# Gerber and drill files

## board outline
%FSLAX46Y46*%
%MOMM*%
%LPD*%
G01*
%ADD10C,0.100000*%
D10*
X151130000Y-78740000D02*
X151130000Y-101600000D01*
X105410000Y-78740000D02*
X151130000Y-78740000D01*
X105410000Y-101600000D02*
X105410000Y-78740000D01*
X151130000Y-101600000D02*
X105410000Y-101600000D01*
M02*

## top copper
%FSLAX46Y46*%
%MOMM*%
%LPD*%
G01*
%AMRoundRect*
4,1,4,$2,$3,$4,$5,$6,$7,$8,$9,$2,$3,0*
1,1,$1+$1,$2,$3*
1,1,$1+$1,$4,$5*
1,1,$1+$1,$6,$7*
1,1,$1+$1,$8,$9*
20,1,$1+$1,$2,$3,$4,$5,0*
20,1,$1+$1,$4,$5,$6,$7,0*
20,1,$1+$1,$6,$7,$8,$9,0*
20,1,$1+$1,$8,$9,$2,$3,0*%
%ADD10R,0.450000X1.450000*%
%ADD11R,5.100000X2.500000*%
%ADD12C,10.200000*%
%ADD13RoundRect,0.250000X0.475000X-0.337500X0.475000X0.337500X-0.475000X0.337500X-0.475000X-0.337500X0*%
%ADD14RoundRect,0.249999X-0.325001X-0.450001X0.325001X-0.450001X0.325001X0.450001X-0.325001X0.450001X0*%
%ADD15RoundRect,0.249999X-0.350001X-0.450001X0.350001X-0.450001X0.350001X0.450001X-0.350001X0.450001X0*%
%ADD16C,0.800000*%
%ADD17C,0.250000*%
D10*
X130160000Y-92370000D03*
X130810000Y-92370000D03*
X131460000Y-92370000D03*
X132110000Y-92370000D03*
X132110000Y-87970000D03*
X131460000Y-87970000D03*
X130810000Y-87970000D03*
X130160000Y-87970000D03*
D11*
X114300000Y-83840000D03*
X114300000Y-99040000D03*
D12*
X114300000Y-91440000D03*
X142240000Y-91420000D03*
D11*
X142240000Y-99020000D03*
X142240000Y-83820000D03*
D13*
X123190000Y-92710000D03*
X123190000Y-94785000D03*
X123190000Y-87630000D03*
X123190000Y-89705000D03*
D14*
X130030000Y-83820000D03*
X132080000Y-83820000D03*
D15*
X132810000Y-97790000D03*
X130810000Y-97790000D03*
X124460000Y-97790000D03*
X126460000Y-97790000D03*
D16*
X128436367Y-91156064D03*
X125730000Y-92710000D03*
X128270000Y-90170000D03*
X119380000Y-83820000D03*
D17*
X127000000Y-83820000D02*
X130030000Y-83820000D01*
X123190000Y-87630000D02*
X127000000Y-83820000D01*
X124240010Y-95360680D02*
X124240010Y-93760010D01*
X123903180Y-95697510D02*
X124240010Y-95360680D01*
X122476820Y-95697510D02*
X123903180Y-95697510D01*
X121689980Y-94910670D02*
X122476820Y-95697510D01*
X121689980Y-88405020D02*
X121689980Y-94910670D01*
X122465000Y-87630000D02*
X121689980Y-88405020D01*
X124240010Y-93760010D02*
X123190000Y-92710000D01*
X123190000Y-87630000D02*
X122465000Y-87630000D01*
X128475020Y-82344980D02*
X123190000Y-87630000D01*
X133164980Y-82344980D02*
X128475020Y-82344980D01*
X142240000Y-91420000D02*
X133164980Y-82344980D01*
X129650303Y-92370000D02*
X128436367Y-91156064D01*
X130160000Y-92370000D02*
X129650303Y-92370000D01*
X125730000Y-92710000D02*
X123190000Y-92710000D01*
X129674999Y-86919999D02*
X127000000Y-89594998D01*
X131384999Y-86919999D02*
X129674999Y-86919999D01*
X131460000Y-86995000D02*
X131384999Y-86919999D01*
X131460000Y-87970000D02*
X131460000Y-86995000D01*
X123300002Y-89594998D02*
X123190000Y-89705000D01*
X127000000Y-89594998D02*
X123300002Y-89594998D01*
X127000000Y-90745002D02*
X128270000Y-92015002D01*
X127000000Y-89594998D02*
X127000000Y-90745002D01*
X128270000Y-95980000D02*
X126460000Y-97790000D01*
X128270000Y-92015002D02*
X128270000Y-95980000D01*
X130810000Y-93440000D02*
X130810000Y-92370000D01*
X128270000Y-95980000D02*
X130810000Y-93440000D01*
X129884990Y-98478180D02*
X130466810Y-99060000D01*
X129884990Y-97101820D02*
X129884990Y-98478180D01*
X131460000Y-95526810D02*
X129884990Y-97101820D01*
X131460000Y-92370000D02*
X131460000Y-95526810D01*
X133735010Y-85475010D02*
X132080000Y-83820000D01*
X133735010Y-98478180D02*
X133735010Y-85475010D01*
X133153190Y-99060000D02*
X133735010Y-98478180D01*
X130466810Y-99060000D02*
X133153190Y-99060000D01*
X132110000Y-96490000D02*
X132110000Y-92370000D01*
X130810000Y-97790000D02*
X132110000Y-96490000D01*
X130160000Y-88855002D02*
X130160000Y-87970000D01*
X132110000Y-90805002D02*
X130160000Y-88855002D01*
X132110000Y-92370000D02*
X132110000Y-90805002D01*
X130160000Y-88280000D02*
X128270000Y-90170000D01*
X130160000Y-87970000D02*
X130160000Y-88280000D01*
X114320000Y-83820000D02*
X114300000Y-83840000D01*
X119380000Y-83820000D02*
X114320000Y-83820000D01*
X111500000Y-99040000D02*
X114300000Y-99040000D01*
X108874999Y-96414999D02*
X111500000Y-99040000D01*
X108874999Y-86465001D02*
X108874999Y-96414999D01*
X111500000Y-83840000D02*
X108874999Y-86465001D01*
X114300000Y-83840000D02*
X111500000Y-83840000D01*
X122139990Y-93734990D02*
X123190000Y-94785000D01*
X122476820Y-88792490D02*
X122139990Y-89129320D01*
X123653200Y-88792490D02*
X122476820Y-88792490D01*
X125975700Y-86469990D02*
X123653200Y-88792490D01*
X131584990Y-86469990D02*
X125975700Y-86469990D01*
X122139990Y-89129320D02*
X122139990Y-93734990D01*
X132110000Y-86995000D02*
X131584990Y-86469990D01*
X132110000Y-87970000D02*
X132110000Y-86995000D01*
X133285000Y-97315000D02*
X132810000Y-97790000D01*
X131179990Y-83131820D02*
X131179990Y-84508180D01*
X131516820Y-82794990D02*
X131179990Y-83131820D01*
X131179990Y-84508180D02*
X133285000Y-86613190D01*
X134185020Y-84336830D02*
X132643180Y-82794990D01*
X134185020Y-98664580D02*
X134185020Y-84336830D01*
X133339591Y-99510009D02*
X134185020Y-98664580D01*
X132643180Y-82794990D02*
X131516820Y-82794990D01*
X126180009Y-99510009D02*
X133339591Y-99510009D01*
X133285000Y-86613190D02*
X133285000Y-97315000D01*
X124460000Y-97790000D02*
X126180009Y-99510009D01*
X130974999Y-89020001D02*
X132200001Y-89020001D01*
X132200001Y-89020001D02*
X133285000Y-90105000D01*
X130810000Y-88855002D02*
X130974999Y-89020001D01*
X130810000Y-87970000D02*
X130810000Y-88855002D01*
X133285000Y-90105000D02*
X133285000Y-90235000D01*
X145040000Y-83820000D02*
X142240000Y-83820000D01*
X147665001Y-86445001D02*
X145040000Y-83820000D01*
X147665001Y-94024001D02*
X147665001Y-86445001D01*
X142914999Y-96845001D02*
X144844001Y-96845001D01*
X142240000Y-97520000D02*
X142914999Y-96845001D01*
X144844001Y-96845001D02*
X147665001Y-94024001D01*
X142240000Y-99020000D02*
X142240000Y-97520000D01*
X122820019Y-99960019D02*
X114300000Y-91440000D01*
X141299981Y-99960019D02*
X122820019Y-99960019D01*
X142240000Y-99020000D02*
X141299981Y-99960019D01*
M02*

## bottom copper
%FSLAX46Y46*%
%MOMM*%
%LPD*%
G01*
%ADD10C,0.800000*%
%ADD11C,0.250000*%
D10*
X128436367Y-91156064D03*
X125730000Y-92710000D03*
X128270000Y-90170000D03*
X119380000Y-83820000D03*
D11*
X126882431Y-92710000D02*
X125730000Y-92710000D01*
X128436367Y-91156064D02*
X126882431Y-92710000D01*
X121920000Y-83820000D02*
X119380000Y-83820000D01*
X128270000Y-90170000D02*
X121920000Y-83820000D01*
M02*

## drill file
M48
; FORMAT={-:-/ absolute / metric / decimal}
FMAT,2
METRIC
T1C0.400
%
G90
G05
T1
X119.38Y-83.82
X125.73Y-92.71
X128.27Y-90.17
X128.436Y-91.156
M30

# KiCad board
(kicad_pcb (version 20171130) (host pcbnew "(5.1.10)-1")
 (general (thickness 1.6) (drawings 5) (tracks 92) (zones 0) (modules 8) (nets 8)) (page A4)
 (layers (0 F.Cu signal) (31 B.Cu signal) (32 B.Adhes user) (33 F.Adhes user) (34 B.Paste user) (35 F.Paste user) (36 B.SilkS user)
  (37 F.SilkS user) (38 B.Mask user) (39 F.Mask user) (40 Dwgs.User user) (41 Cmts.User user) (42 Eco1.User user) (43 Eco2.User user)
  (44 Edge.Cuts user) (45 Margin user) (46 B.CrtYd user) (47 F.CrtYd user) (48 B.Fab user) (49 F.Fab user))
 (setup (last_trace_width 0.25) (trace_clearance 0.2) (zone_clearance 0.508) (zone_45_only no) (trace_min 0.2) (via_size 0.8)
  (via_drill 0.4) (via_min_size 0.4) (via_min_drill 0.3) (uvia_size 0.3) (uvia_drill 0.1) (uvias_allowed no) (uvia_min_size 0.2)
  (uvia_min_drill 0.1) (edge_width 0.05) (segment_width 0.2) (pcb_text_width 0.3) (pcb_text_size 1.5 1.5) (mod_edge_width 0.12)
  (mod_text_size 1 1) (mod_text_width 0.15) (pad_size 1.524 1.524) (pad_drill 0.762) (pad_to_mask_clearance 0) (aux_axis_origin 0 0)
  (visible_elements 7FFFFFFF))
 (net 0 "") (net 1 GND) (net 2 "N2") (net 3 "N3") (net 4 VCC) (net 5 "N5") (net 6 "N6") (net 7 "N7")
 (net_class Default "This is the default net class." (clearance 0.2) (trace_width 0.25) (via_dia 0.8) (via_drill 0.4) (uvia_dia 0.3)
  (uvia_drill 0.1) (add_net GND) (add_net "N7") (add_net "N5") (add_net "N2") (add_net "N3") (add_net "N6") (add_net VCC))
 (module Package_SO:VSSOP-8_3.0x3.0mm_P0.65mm (layer F.Cu) (at 131.135 90.17 90)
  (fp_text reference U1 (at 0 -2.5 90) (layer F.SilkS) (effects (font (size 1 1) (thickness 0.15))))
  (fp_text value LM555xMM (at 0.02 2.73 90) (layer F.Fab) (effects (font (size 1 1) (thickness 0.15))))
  (pad 1 smd rect (at -2.2 -0.975) (size 0.45 1.45) (layers F.Cu F.Paste F.Mask) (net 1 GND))
  (pad 2 smd rect (at -2.2 -0.325) (size 0.45 1.45) (layers F.Cu F.Paste F.Mask) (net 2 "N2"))
  (pad 3 smd rect (at -2.2 0.325) (size 0.45 1.45) (layers F.Cu F.Paste F.Mask) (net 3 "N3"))
  (pad 4 smd rect (at -2.2 0.975) (size 0.45 1.45) (layers F.Cu F.Paste F.Mask) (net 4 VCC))
  (pad 5 smd rect (at 2.2 0.975) (size 0.45 1.45) (layers F.Cu F.Paste F.Mask) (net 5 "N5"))
  (pad 6 smd rect (at 2.2 0.325) (size 0.45 1.45) (layers F.Cu F.Paste F.Mask) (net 2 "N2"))
  (pad 7 smd rect (at 2.2 -0.325) (size 0.45 1.45) (layers F.Cu F.Paste F.Mask) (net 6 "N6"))
  (pad 8 smd rect (at 2.2 -0.975) (size 0.45 1.45) (layers F.Cu F.Paste F.Mask) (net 4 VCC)))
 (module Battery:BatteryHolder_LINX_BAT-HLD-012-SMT (layer F.Cu) (at 114.3 91.44 270)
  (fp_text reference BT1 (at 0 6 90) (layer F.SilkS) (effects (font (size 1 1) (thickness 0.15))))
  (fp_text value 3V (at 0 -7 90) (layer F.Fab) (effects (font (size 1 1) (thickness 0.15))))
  (pad 1 smd rect (at -7.6 0 270) (size 2.5 5.1) (layers F.Cu F.Paste F.Mask) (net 4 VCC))
  (pad 1 smd rect (at 7.6 0 270) (size 2.5 5.1) (layers F.Cu F.Paste F.Mask) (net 4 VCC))
  (pad 2 smd circle (at 0 0 270) (size 10.2 10.2) (layers F.Cu F.Mask) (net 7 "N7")))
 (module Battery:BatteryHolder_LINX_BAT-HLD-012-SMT (layer F.Cu) (at 142.24 91.42 270)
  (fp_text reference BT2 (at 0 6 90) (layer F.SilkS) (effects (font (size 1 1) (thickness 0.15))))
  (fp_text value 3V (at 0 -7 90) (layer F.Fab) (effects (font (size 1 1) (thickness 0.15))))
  (pad 2 smd circle (at 0 0 270) (size 10.2 10.2) (layers F.Cu F.Mask) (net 1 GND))
  (pad 1 smd rect (at 7.6 0 270) (size 2.5 5.1) (layers F.Cu F.Paste F.Mask) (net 7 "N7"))
  (pad 1 smd rect (at -7.6 0 270) (size 2.5 5.1) (layers F.Cu F.Paste F.Mask) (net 7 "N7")))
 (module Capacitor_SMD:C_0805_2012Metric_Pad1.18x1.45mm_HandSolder (layer F.Cu) (at 123.19 93.7475 90)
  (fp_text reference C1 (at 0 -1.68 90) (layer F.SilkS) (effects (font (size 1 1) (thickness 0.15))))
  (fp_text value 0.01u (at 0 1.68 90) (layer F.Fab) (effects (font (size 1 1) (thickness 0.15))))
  (pad 2 smd roundrect (at 1.0375 0 90) (size 1.175 1.45) (layers F.Cu F.Paste F.Mask) (roundrect_rratio 0.2127659574468085) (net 1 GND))
  (pad 1 smd roundrect (at -1.0375 0 90) (size 1.175 1.45) (layers F.Cu F.Paste F.Mask) (roundrect_rratio 0.2127659574468085) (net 5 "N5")))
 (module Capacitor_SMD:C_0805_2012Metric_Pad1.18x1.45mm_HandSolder (layer F.Cu) (at 123.19 88.6675 90)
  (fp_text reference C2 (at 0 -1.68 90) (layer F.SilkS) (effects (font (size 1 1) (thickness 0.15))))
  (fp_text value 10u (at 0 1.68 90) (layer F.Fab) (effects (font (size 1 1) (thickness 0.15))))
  (pad 2 smd roundrect (at 1.0375 0 90) (size 1.175 1.45) (layers F.Cu F.Paste F.Mask) (roundrect_rratio 0.2127659574468085) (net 1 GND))
  (pad 1 smd roundrect (at -1.0375 0 90) (size 1.175 1.45) (layers F.Cu F.Paste F.Mask) (roundrect_rratio 0.2127659574468085) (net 2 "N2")))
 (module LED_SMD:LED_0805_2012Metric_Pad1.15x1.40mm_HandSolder (layer F.Cu) (at 131.055 83.82)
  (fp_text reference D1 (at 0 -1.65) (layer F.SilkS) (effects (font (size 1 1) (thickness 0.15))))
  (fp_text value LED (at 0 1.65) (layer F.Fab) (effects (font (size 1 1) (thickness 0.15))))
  (pad 1 smd roundrect (at -1.025 0) (size 1.15 1.4) (layers F.Cu F.Paste F.Mask) (roundrect_rratio 0.2173904347826087) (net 1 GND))
  (pad 2 smd roundrect (at 1.025 0) (size 1.15 1.4) (layers F.Cu F.Paste F.Mask) (roundrect_rratio 0.2173904347826087) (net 3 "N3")))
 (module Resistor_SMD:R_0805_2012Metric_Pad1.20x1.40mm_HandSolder (layer F.Cu) (at 131.81 97.79)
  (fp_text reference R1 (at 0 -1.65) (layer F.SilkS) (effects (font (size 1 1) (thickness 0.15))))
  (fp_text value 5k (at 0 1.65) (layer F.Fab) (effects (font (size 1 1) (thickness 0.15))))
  (pad 2 smd roundrect (at 1 0) (size 1.2 1.4) (layers F.Cu F.Paste F.Mask) (roundrect_rratio 0.2083325) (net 6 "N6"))
  (pad 1 smd roundrect (at -1 0) (size 1.2 1.4) (layers F.Cu F.Paste F.Mask) (roundrect_rratio 0.2083325) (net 4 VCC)))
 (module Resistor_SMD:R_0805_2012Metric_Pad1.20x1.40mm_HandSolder (layer F.Cu) (at 125.46 97.79)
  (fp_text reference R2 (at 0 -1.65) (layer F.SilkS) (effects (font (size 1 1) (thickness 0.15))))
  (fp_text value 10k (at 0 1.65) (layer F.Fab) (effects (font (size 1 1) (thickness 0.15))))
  (pad 1 smd roundrect (at -1 0) (size 1.2 1.4) (layers F.Cu F.Paste F.Mask) (roundrect_rratio 0.2083325) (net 6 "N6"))
  (pad 2 smd roundrect (at 1 0) (size 1.2 1.4) (layers F.Cu F.Paste F.Mask) (roundrect_rratio 0.2083325) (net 2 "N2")))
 (gr_line (start 151.13 78.74) (end 151.13 101.6) (layer Edge.Cuts) (width 0.1))
 (gr_line (start 105.41 78.74) (end 151.13 78.74) (layer Edge.Cuts) (width 0.1))
 (gr_line (start 105.41 101.6) (end 105.41 78.74) (layer Edge.Cuts) (width 0.1))
 (gr_line (start 151.13 101.6) (end 105.41 101.6) (layer Edge.Cuts) (width 0.1))
 (segment (start 127 83.82) (end 130.03 83.82) (width 0.25) (layer F.Cu) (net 1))
 (segment (start 123.19 87.63) (end 127 83.82) (width 0.25) (layer F.Cu) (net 1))
 (segment (start 124.24001 95.36068) (end 124.24001 93.76001) (width 0.25) (layer F.Cu) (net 1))
 (segment (start 123.90318 95.69751) (end 124.24001 95.36068) (width 0.25) (layer F.Cu) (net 1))
 (segment (start 122.47682 95.69751) (end 123.90318 95.69751) (width 0.25) (layer F.Cu) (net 1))
 (segment (start 121.68998 94.91067) (end 122.47682 95.69751) (width 0.25) (layer F.Cu) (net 1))
 (segment (start 121.68998 88.40502) (end 121.68998 94.91067) (width 0.25) (layer F.Cu) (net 1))
 (segment (start 122.465 87.63) (end 121.68998 88.40502) (width 0.25) (layer F.Cu) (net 1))
 (segment (start 124.24001 93.76001) (end 123.19 92.71) (width 0.25) (layer F.Cu) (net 1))
 (segment (start 123.19 87.63) (end 122.465 87.63) (width 0.25) (layer F.Cu) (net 1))
 (segment (start 128.47502 82.34498) (end 123.19 87.63) (width 0.25) (layer F.Cu) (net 1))
 (segment (start 133.16498 82.34498) (end 128.47502 82.34498) (width 0.25) (layer F.Cu) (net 1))
 (segment (start 142.24 91.42) (end 133.16498 82.34498) (width 0.25) (layer F.Cu) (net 1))
 (via (at 128.436367 91.156064) (size 0.8) (drill 0.4) (layers F.Cu B.Cu) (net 1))
 (segment (start 129.650303 92.37) (end 128.436367 91.156064) (width 0.25) (layer F.Cu) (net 1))
 (segment (start 130.16 92.37) (end 129.650303 92.37) (width 0.25) (layer F.Cu) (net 1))
 (via (at 125.73 92.71) (size 0.8) (drill 0.4) (layers F.Cu B.Cu) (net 1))
 (segment (start 126.882431 92.71) (end 125.73 92.71) (width 0.25) (layer B.Cu) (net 1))
 (segment (start 128.436367 91.156064) (end 126.882431 92.71) (width 0.25) (layer B.Cu) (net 1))
 (segment (start 125.73 92.71) (end 123.19 92.71) (width 0.25) (layer F.Cu) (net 1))
 (segment (start 129.674999 86.919999) (end 127 89.594998) (width 0.25) (layer F.Cu) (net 2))
 (segment (start 131.384999 86.919999) (end 129.674999 86.919999) (width 0.25) (layer F.Cu) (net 2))
 (segment (start 131.46 86.995) (end 131.384999 86.919999) (width 0.25) (layer F.Cu) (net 2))
 (segment (start 131.46 87.97) (end 131.46 86.995) (width 0.25) (layer F.Cu) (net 2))
 (segment (start 123.300002 89.594998) (end 123.19 89.705) (width 0.25) (layer F.Cu) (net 2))
 (segment (start 127 89.594998) (end 123.300002 89.594998) (width 0.25) (layer F.Cu) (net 2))
 (segment (start 127 90.745002) (end 128.27 92.015002) (width 0.25) (layer F.Cu) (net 2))
 (segment (start 127 89.594998) (end 127 90.745002) (width 0.25) (layer F.Cu) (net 2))
 (segment (start 128.27 95.98) (end 126.46 97.79) (width 0.25) (layer F.Cu) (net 2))
 (segment (start 128.27 92.015002) (end 128.27 95.98) (width 0.25) (layer F.Cu) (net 2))
 (segment (start 130.81 93.44) (end 130.81 92.37) (width 0.25) (layer F.Cu) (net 2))
 (segment (start 128.27 95.98) (end 130.81 93.44) (width 0.25) (layer F.Cu) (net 2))
 (segment (start 129.88499 98.47818) (end 130.46681 99.06) (width 0.25) (layer F.Cu) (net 3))
 (segment (start 129.88499 97.10182) (end 129.88499 98.47818) (width 0.25) (layer F.Cu) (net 3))
 (segment (start 131.46 95.52681) (end 129.88499 97.10182) (width 0.25) (layer F.Cu) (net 3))
 (segment (start 131.46 92.37) (end 131.46 95.52681) (width 0.25) (layer F.Cu) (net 3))
 (segment (start 133.73501 85.47501) (end 132.08 83.82) (width 0.25) (layer F.Cu) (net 3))
 (segment (start 133.73501 98.47818) (end 133.73501 85.47501) (width 0.25) (layer F.Cu) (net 3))
 (segment (start 133.15319 99.06) (end 133.73501 98.47818) (width 0.25) (layer F.Cu) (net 3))
 (segment (start 130.46681 99.06) (end 133.15319 99.06) (width 0.25) (layer F.Cu) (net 3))
 (segment (start 132.11 96.49) (end 132.11 92.37) (width 0.25) (layer F.Cu) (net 4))
 (segment (start 130.81 97.79) (end 132.11 96.49) (width 0.25) (layer F.Cu) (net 4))
 (segment (start 130.16 88.855002) (end 130.16 87.97) (width 0.25) (layer F.Cu) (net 4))
 (segment (start 132.11 90.805002) (end 130.16 88.855002) (width 0.25) (layer F.Cu) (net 4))
 (segment (start 132.11 92.37) (end 132.11 90.805002) (width 0.25) (layer F.Cu) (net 4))
 (via (at 128.27 90.17) (size 0.8) (drill 0.4) (layers F.Cu B.Cu) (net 4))
 (segment (start 130.16 88.28) (end 128.27 90.17) (width 0.25) (layer F.Cu) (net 4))
 (segment (start 130.16 87.97) (end 130.16 88.28) (width 0.25) (layer F.Cu) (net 4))
 (via (at 119.38 83.82) (size 0.8) (drill 0.4) (layers F.Cu B.Cu) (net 4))
 (segment (start 121.92 83.82) (end 119.38 83.82) (width 0.25) (layer B.Cu) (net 4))
 (segment (start 128.27 90.17) (end 121.92 83.82) (width 0.25) (layer B.Cu) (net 4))
 (segment (start 114.32 83.82) (end 114.3 83.84) (width 0.25) (layer F.Cu) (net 4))
 (segment (start 119.38 83.82) (end 114.32 83.82) (width 0.25) (layer F.Cu) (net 4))
 (segment (start 111.5 99.04) (end 114.3 99.04) (width 0.25) (layer F.Cu) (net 4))
 (segment (start 108.874999 96.414999) (end 111.5 99.04) (width 0.25) (layer F.Cu) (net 4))
 (segment (start 108.874999 86.465001) (end 108.874999 96.414999) (width 0.25) (layer F.Cu) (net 4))
 (segment (start 111.5 83.84) (end 108.874999 86.465001) (width 0.25) (layer F.Cu) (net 4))
 (segment (start 114.3 83.84) (end 111.5 83.84) (width 0.25) (layer F.Cu) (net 4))
 (segment (start 122.13999 93.73499) (end 123.19 94.785) (width 0.25) (layer F.Cu) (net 5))
 (segment (start 122.47682 88.79249) (end 122.13999 89.12932) (width 0.25) (layer F.Cu) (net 5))
 (segment (start 123.6532 88.79249) (end 122.47682 88.79249) (width 0.25) (layer F.Cu) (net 5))
 (segment (start 125.9757 86.46999) (end 123.6532 88.79249) (width 0.25) (layer F.Cu) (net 5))
 (segment (start 131.58499 86.46999) (end 125.9757 86.46999) (width 0.25) (layer F.Cu) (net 5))
 (segment (start 122.13999 89.12932) (end 122.13999 93.73499) (width 0.25) (layer F.Cu) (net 5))
 (segment (start 132.11 86.995) (end 131.58499 86.46999) (width 0.25) (layer F.Cu) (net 5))
 (segment (start 132.11 87.97) (end 132.11 86.995) (width 0.25) (layer F.Cu) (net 5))
 (segment (start 133.285 97.315) (end 132.81 97.79) (width 0.25) (layer F.Cu) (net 6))
 (segment (start 131.17999 83.13182) (end 131.17999 84.50818) (width 0.25) (layer F.Cu) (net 6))
 (segment (start 131.51682 82.79499) (end 131.17999 83.13182) (width 0.25) (layer F.Cu) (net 6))
 (segment (start 131.17999 84.50818) (end 133.285 86.61319) (width 0.25) (layer F.Cu) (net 6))
 (segment (start 134.18502 84.33683) (end 132.64318 82.79499) (width 0.25) (layer F.Cu) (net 6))
 (segment (start 134.18502 98.66458) (end 134.18502 84.33683) (width 0.25) (layer F.Cu) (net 6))
 (segment (start 133.339591 99.510009) (end 134.18502 98.66458) (width 0.25) (layer F.Cu) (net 6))
 (segment (start 132.64318 82.79499) (end 131.51682 82.79499) (width 0.25) (layer F.Cu) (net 6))
 (segment (start 126.180009 99.510009) (end 133.339591 99.510009) (width 0.25) (layer F.Cu) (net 6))
 (segment (start 133.285 86.61319) (end 133.285 97.315) (width 0.25) (layer F.Cu) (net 6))
 (segment (start 124.46 97.79) (end 126.180009 99.510009) (width 0.25) (layer F.Cu) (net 6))
 (segment (start 130.974999 89.020001) (end 132.200001 89.020001) (width 0.25) (layer F.Cu) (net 6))
 (segment (start 132.200001 89.020001) (end 133.285 90.105) (width 0.25) (layer F.Cu) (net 6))
 (segment (start 130.81 88.855002) (end 130.974999 89.020001) (width 0.25) (layer F.Cu) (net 6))
 (segment (start 130.81 87.97) (end 130.81 88.855002) (width 0.25) (layer F.Cu) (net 6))
 (segment (start 133.285 90.105) (end 133.285 90.235) (width 0.25) (layer F.Cu) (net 6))
 (segment (start 145.04 83.82) (end 142.24 83.82) (width 0.25) (layer F.Cu) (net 7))
 (segment (start 147.665001 86.445001) (end 145.04 83.82) (width 0.25) (layer F.Cu) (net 7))
 (segment (start 147.665001 94.024001) (end 147.665001 86.445001) (width 0.25) (layer F.Cu) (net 7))
 (segment (start 142.914999 96.845001) (end 144.844001 96.845001) (width 0.25) (layer F.Cu) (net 7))
 (segment (start 142.24 97.52) (end 142.914999 96.845001) (width 0.25) (layer F.Cu) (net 7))
 (segment (start 144.844001 96.845001) (end 147.665001 94.024001) (width 0.25) (layer F.Cu) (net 7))
 (segment (start 142.24 99.02) (end 142.24 97.52) (width 0.25) (layer F.Cu) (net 7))
 (segment (start 122.820019 99.960019) (end 114.3 91.44) (width 0.25) (layer F.Cu) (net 7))
 (segment (start 141.299981 99.960019) (end 122.820019 99.960019) (width 0.25) (layer F.Cu) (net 7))
 (segment (start 142.24 99.02) (end 141.299981 99.960019) (width 0.25) (layer F.Cu) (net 7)))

